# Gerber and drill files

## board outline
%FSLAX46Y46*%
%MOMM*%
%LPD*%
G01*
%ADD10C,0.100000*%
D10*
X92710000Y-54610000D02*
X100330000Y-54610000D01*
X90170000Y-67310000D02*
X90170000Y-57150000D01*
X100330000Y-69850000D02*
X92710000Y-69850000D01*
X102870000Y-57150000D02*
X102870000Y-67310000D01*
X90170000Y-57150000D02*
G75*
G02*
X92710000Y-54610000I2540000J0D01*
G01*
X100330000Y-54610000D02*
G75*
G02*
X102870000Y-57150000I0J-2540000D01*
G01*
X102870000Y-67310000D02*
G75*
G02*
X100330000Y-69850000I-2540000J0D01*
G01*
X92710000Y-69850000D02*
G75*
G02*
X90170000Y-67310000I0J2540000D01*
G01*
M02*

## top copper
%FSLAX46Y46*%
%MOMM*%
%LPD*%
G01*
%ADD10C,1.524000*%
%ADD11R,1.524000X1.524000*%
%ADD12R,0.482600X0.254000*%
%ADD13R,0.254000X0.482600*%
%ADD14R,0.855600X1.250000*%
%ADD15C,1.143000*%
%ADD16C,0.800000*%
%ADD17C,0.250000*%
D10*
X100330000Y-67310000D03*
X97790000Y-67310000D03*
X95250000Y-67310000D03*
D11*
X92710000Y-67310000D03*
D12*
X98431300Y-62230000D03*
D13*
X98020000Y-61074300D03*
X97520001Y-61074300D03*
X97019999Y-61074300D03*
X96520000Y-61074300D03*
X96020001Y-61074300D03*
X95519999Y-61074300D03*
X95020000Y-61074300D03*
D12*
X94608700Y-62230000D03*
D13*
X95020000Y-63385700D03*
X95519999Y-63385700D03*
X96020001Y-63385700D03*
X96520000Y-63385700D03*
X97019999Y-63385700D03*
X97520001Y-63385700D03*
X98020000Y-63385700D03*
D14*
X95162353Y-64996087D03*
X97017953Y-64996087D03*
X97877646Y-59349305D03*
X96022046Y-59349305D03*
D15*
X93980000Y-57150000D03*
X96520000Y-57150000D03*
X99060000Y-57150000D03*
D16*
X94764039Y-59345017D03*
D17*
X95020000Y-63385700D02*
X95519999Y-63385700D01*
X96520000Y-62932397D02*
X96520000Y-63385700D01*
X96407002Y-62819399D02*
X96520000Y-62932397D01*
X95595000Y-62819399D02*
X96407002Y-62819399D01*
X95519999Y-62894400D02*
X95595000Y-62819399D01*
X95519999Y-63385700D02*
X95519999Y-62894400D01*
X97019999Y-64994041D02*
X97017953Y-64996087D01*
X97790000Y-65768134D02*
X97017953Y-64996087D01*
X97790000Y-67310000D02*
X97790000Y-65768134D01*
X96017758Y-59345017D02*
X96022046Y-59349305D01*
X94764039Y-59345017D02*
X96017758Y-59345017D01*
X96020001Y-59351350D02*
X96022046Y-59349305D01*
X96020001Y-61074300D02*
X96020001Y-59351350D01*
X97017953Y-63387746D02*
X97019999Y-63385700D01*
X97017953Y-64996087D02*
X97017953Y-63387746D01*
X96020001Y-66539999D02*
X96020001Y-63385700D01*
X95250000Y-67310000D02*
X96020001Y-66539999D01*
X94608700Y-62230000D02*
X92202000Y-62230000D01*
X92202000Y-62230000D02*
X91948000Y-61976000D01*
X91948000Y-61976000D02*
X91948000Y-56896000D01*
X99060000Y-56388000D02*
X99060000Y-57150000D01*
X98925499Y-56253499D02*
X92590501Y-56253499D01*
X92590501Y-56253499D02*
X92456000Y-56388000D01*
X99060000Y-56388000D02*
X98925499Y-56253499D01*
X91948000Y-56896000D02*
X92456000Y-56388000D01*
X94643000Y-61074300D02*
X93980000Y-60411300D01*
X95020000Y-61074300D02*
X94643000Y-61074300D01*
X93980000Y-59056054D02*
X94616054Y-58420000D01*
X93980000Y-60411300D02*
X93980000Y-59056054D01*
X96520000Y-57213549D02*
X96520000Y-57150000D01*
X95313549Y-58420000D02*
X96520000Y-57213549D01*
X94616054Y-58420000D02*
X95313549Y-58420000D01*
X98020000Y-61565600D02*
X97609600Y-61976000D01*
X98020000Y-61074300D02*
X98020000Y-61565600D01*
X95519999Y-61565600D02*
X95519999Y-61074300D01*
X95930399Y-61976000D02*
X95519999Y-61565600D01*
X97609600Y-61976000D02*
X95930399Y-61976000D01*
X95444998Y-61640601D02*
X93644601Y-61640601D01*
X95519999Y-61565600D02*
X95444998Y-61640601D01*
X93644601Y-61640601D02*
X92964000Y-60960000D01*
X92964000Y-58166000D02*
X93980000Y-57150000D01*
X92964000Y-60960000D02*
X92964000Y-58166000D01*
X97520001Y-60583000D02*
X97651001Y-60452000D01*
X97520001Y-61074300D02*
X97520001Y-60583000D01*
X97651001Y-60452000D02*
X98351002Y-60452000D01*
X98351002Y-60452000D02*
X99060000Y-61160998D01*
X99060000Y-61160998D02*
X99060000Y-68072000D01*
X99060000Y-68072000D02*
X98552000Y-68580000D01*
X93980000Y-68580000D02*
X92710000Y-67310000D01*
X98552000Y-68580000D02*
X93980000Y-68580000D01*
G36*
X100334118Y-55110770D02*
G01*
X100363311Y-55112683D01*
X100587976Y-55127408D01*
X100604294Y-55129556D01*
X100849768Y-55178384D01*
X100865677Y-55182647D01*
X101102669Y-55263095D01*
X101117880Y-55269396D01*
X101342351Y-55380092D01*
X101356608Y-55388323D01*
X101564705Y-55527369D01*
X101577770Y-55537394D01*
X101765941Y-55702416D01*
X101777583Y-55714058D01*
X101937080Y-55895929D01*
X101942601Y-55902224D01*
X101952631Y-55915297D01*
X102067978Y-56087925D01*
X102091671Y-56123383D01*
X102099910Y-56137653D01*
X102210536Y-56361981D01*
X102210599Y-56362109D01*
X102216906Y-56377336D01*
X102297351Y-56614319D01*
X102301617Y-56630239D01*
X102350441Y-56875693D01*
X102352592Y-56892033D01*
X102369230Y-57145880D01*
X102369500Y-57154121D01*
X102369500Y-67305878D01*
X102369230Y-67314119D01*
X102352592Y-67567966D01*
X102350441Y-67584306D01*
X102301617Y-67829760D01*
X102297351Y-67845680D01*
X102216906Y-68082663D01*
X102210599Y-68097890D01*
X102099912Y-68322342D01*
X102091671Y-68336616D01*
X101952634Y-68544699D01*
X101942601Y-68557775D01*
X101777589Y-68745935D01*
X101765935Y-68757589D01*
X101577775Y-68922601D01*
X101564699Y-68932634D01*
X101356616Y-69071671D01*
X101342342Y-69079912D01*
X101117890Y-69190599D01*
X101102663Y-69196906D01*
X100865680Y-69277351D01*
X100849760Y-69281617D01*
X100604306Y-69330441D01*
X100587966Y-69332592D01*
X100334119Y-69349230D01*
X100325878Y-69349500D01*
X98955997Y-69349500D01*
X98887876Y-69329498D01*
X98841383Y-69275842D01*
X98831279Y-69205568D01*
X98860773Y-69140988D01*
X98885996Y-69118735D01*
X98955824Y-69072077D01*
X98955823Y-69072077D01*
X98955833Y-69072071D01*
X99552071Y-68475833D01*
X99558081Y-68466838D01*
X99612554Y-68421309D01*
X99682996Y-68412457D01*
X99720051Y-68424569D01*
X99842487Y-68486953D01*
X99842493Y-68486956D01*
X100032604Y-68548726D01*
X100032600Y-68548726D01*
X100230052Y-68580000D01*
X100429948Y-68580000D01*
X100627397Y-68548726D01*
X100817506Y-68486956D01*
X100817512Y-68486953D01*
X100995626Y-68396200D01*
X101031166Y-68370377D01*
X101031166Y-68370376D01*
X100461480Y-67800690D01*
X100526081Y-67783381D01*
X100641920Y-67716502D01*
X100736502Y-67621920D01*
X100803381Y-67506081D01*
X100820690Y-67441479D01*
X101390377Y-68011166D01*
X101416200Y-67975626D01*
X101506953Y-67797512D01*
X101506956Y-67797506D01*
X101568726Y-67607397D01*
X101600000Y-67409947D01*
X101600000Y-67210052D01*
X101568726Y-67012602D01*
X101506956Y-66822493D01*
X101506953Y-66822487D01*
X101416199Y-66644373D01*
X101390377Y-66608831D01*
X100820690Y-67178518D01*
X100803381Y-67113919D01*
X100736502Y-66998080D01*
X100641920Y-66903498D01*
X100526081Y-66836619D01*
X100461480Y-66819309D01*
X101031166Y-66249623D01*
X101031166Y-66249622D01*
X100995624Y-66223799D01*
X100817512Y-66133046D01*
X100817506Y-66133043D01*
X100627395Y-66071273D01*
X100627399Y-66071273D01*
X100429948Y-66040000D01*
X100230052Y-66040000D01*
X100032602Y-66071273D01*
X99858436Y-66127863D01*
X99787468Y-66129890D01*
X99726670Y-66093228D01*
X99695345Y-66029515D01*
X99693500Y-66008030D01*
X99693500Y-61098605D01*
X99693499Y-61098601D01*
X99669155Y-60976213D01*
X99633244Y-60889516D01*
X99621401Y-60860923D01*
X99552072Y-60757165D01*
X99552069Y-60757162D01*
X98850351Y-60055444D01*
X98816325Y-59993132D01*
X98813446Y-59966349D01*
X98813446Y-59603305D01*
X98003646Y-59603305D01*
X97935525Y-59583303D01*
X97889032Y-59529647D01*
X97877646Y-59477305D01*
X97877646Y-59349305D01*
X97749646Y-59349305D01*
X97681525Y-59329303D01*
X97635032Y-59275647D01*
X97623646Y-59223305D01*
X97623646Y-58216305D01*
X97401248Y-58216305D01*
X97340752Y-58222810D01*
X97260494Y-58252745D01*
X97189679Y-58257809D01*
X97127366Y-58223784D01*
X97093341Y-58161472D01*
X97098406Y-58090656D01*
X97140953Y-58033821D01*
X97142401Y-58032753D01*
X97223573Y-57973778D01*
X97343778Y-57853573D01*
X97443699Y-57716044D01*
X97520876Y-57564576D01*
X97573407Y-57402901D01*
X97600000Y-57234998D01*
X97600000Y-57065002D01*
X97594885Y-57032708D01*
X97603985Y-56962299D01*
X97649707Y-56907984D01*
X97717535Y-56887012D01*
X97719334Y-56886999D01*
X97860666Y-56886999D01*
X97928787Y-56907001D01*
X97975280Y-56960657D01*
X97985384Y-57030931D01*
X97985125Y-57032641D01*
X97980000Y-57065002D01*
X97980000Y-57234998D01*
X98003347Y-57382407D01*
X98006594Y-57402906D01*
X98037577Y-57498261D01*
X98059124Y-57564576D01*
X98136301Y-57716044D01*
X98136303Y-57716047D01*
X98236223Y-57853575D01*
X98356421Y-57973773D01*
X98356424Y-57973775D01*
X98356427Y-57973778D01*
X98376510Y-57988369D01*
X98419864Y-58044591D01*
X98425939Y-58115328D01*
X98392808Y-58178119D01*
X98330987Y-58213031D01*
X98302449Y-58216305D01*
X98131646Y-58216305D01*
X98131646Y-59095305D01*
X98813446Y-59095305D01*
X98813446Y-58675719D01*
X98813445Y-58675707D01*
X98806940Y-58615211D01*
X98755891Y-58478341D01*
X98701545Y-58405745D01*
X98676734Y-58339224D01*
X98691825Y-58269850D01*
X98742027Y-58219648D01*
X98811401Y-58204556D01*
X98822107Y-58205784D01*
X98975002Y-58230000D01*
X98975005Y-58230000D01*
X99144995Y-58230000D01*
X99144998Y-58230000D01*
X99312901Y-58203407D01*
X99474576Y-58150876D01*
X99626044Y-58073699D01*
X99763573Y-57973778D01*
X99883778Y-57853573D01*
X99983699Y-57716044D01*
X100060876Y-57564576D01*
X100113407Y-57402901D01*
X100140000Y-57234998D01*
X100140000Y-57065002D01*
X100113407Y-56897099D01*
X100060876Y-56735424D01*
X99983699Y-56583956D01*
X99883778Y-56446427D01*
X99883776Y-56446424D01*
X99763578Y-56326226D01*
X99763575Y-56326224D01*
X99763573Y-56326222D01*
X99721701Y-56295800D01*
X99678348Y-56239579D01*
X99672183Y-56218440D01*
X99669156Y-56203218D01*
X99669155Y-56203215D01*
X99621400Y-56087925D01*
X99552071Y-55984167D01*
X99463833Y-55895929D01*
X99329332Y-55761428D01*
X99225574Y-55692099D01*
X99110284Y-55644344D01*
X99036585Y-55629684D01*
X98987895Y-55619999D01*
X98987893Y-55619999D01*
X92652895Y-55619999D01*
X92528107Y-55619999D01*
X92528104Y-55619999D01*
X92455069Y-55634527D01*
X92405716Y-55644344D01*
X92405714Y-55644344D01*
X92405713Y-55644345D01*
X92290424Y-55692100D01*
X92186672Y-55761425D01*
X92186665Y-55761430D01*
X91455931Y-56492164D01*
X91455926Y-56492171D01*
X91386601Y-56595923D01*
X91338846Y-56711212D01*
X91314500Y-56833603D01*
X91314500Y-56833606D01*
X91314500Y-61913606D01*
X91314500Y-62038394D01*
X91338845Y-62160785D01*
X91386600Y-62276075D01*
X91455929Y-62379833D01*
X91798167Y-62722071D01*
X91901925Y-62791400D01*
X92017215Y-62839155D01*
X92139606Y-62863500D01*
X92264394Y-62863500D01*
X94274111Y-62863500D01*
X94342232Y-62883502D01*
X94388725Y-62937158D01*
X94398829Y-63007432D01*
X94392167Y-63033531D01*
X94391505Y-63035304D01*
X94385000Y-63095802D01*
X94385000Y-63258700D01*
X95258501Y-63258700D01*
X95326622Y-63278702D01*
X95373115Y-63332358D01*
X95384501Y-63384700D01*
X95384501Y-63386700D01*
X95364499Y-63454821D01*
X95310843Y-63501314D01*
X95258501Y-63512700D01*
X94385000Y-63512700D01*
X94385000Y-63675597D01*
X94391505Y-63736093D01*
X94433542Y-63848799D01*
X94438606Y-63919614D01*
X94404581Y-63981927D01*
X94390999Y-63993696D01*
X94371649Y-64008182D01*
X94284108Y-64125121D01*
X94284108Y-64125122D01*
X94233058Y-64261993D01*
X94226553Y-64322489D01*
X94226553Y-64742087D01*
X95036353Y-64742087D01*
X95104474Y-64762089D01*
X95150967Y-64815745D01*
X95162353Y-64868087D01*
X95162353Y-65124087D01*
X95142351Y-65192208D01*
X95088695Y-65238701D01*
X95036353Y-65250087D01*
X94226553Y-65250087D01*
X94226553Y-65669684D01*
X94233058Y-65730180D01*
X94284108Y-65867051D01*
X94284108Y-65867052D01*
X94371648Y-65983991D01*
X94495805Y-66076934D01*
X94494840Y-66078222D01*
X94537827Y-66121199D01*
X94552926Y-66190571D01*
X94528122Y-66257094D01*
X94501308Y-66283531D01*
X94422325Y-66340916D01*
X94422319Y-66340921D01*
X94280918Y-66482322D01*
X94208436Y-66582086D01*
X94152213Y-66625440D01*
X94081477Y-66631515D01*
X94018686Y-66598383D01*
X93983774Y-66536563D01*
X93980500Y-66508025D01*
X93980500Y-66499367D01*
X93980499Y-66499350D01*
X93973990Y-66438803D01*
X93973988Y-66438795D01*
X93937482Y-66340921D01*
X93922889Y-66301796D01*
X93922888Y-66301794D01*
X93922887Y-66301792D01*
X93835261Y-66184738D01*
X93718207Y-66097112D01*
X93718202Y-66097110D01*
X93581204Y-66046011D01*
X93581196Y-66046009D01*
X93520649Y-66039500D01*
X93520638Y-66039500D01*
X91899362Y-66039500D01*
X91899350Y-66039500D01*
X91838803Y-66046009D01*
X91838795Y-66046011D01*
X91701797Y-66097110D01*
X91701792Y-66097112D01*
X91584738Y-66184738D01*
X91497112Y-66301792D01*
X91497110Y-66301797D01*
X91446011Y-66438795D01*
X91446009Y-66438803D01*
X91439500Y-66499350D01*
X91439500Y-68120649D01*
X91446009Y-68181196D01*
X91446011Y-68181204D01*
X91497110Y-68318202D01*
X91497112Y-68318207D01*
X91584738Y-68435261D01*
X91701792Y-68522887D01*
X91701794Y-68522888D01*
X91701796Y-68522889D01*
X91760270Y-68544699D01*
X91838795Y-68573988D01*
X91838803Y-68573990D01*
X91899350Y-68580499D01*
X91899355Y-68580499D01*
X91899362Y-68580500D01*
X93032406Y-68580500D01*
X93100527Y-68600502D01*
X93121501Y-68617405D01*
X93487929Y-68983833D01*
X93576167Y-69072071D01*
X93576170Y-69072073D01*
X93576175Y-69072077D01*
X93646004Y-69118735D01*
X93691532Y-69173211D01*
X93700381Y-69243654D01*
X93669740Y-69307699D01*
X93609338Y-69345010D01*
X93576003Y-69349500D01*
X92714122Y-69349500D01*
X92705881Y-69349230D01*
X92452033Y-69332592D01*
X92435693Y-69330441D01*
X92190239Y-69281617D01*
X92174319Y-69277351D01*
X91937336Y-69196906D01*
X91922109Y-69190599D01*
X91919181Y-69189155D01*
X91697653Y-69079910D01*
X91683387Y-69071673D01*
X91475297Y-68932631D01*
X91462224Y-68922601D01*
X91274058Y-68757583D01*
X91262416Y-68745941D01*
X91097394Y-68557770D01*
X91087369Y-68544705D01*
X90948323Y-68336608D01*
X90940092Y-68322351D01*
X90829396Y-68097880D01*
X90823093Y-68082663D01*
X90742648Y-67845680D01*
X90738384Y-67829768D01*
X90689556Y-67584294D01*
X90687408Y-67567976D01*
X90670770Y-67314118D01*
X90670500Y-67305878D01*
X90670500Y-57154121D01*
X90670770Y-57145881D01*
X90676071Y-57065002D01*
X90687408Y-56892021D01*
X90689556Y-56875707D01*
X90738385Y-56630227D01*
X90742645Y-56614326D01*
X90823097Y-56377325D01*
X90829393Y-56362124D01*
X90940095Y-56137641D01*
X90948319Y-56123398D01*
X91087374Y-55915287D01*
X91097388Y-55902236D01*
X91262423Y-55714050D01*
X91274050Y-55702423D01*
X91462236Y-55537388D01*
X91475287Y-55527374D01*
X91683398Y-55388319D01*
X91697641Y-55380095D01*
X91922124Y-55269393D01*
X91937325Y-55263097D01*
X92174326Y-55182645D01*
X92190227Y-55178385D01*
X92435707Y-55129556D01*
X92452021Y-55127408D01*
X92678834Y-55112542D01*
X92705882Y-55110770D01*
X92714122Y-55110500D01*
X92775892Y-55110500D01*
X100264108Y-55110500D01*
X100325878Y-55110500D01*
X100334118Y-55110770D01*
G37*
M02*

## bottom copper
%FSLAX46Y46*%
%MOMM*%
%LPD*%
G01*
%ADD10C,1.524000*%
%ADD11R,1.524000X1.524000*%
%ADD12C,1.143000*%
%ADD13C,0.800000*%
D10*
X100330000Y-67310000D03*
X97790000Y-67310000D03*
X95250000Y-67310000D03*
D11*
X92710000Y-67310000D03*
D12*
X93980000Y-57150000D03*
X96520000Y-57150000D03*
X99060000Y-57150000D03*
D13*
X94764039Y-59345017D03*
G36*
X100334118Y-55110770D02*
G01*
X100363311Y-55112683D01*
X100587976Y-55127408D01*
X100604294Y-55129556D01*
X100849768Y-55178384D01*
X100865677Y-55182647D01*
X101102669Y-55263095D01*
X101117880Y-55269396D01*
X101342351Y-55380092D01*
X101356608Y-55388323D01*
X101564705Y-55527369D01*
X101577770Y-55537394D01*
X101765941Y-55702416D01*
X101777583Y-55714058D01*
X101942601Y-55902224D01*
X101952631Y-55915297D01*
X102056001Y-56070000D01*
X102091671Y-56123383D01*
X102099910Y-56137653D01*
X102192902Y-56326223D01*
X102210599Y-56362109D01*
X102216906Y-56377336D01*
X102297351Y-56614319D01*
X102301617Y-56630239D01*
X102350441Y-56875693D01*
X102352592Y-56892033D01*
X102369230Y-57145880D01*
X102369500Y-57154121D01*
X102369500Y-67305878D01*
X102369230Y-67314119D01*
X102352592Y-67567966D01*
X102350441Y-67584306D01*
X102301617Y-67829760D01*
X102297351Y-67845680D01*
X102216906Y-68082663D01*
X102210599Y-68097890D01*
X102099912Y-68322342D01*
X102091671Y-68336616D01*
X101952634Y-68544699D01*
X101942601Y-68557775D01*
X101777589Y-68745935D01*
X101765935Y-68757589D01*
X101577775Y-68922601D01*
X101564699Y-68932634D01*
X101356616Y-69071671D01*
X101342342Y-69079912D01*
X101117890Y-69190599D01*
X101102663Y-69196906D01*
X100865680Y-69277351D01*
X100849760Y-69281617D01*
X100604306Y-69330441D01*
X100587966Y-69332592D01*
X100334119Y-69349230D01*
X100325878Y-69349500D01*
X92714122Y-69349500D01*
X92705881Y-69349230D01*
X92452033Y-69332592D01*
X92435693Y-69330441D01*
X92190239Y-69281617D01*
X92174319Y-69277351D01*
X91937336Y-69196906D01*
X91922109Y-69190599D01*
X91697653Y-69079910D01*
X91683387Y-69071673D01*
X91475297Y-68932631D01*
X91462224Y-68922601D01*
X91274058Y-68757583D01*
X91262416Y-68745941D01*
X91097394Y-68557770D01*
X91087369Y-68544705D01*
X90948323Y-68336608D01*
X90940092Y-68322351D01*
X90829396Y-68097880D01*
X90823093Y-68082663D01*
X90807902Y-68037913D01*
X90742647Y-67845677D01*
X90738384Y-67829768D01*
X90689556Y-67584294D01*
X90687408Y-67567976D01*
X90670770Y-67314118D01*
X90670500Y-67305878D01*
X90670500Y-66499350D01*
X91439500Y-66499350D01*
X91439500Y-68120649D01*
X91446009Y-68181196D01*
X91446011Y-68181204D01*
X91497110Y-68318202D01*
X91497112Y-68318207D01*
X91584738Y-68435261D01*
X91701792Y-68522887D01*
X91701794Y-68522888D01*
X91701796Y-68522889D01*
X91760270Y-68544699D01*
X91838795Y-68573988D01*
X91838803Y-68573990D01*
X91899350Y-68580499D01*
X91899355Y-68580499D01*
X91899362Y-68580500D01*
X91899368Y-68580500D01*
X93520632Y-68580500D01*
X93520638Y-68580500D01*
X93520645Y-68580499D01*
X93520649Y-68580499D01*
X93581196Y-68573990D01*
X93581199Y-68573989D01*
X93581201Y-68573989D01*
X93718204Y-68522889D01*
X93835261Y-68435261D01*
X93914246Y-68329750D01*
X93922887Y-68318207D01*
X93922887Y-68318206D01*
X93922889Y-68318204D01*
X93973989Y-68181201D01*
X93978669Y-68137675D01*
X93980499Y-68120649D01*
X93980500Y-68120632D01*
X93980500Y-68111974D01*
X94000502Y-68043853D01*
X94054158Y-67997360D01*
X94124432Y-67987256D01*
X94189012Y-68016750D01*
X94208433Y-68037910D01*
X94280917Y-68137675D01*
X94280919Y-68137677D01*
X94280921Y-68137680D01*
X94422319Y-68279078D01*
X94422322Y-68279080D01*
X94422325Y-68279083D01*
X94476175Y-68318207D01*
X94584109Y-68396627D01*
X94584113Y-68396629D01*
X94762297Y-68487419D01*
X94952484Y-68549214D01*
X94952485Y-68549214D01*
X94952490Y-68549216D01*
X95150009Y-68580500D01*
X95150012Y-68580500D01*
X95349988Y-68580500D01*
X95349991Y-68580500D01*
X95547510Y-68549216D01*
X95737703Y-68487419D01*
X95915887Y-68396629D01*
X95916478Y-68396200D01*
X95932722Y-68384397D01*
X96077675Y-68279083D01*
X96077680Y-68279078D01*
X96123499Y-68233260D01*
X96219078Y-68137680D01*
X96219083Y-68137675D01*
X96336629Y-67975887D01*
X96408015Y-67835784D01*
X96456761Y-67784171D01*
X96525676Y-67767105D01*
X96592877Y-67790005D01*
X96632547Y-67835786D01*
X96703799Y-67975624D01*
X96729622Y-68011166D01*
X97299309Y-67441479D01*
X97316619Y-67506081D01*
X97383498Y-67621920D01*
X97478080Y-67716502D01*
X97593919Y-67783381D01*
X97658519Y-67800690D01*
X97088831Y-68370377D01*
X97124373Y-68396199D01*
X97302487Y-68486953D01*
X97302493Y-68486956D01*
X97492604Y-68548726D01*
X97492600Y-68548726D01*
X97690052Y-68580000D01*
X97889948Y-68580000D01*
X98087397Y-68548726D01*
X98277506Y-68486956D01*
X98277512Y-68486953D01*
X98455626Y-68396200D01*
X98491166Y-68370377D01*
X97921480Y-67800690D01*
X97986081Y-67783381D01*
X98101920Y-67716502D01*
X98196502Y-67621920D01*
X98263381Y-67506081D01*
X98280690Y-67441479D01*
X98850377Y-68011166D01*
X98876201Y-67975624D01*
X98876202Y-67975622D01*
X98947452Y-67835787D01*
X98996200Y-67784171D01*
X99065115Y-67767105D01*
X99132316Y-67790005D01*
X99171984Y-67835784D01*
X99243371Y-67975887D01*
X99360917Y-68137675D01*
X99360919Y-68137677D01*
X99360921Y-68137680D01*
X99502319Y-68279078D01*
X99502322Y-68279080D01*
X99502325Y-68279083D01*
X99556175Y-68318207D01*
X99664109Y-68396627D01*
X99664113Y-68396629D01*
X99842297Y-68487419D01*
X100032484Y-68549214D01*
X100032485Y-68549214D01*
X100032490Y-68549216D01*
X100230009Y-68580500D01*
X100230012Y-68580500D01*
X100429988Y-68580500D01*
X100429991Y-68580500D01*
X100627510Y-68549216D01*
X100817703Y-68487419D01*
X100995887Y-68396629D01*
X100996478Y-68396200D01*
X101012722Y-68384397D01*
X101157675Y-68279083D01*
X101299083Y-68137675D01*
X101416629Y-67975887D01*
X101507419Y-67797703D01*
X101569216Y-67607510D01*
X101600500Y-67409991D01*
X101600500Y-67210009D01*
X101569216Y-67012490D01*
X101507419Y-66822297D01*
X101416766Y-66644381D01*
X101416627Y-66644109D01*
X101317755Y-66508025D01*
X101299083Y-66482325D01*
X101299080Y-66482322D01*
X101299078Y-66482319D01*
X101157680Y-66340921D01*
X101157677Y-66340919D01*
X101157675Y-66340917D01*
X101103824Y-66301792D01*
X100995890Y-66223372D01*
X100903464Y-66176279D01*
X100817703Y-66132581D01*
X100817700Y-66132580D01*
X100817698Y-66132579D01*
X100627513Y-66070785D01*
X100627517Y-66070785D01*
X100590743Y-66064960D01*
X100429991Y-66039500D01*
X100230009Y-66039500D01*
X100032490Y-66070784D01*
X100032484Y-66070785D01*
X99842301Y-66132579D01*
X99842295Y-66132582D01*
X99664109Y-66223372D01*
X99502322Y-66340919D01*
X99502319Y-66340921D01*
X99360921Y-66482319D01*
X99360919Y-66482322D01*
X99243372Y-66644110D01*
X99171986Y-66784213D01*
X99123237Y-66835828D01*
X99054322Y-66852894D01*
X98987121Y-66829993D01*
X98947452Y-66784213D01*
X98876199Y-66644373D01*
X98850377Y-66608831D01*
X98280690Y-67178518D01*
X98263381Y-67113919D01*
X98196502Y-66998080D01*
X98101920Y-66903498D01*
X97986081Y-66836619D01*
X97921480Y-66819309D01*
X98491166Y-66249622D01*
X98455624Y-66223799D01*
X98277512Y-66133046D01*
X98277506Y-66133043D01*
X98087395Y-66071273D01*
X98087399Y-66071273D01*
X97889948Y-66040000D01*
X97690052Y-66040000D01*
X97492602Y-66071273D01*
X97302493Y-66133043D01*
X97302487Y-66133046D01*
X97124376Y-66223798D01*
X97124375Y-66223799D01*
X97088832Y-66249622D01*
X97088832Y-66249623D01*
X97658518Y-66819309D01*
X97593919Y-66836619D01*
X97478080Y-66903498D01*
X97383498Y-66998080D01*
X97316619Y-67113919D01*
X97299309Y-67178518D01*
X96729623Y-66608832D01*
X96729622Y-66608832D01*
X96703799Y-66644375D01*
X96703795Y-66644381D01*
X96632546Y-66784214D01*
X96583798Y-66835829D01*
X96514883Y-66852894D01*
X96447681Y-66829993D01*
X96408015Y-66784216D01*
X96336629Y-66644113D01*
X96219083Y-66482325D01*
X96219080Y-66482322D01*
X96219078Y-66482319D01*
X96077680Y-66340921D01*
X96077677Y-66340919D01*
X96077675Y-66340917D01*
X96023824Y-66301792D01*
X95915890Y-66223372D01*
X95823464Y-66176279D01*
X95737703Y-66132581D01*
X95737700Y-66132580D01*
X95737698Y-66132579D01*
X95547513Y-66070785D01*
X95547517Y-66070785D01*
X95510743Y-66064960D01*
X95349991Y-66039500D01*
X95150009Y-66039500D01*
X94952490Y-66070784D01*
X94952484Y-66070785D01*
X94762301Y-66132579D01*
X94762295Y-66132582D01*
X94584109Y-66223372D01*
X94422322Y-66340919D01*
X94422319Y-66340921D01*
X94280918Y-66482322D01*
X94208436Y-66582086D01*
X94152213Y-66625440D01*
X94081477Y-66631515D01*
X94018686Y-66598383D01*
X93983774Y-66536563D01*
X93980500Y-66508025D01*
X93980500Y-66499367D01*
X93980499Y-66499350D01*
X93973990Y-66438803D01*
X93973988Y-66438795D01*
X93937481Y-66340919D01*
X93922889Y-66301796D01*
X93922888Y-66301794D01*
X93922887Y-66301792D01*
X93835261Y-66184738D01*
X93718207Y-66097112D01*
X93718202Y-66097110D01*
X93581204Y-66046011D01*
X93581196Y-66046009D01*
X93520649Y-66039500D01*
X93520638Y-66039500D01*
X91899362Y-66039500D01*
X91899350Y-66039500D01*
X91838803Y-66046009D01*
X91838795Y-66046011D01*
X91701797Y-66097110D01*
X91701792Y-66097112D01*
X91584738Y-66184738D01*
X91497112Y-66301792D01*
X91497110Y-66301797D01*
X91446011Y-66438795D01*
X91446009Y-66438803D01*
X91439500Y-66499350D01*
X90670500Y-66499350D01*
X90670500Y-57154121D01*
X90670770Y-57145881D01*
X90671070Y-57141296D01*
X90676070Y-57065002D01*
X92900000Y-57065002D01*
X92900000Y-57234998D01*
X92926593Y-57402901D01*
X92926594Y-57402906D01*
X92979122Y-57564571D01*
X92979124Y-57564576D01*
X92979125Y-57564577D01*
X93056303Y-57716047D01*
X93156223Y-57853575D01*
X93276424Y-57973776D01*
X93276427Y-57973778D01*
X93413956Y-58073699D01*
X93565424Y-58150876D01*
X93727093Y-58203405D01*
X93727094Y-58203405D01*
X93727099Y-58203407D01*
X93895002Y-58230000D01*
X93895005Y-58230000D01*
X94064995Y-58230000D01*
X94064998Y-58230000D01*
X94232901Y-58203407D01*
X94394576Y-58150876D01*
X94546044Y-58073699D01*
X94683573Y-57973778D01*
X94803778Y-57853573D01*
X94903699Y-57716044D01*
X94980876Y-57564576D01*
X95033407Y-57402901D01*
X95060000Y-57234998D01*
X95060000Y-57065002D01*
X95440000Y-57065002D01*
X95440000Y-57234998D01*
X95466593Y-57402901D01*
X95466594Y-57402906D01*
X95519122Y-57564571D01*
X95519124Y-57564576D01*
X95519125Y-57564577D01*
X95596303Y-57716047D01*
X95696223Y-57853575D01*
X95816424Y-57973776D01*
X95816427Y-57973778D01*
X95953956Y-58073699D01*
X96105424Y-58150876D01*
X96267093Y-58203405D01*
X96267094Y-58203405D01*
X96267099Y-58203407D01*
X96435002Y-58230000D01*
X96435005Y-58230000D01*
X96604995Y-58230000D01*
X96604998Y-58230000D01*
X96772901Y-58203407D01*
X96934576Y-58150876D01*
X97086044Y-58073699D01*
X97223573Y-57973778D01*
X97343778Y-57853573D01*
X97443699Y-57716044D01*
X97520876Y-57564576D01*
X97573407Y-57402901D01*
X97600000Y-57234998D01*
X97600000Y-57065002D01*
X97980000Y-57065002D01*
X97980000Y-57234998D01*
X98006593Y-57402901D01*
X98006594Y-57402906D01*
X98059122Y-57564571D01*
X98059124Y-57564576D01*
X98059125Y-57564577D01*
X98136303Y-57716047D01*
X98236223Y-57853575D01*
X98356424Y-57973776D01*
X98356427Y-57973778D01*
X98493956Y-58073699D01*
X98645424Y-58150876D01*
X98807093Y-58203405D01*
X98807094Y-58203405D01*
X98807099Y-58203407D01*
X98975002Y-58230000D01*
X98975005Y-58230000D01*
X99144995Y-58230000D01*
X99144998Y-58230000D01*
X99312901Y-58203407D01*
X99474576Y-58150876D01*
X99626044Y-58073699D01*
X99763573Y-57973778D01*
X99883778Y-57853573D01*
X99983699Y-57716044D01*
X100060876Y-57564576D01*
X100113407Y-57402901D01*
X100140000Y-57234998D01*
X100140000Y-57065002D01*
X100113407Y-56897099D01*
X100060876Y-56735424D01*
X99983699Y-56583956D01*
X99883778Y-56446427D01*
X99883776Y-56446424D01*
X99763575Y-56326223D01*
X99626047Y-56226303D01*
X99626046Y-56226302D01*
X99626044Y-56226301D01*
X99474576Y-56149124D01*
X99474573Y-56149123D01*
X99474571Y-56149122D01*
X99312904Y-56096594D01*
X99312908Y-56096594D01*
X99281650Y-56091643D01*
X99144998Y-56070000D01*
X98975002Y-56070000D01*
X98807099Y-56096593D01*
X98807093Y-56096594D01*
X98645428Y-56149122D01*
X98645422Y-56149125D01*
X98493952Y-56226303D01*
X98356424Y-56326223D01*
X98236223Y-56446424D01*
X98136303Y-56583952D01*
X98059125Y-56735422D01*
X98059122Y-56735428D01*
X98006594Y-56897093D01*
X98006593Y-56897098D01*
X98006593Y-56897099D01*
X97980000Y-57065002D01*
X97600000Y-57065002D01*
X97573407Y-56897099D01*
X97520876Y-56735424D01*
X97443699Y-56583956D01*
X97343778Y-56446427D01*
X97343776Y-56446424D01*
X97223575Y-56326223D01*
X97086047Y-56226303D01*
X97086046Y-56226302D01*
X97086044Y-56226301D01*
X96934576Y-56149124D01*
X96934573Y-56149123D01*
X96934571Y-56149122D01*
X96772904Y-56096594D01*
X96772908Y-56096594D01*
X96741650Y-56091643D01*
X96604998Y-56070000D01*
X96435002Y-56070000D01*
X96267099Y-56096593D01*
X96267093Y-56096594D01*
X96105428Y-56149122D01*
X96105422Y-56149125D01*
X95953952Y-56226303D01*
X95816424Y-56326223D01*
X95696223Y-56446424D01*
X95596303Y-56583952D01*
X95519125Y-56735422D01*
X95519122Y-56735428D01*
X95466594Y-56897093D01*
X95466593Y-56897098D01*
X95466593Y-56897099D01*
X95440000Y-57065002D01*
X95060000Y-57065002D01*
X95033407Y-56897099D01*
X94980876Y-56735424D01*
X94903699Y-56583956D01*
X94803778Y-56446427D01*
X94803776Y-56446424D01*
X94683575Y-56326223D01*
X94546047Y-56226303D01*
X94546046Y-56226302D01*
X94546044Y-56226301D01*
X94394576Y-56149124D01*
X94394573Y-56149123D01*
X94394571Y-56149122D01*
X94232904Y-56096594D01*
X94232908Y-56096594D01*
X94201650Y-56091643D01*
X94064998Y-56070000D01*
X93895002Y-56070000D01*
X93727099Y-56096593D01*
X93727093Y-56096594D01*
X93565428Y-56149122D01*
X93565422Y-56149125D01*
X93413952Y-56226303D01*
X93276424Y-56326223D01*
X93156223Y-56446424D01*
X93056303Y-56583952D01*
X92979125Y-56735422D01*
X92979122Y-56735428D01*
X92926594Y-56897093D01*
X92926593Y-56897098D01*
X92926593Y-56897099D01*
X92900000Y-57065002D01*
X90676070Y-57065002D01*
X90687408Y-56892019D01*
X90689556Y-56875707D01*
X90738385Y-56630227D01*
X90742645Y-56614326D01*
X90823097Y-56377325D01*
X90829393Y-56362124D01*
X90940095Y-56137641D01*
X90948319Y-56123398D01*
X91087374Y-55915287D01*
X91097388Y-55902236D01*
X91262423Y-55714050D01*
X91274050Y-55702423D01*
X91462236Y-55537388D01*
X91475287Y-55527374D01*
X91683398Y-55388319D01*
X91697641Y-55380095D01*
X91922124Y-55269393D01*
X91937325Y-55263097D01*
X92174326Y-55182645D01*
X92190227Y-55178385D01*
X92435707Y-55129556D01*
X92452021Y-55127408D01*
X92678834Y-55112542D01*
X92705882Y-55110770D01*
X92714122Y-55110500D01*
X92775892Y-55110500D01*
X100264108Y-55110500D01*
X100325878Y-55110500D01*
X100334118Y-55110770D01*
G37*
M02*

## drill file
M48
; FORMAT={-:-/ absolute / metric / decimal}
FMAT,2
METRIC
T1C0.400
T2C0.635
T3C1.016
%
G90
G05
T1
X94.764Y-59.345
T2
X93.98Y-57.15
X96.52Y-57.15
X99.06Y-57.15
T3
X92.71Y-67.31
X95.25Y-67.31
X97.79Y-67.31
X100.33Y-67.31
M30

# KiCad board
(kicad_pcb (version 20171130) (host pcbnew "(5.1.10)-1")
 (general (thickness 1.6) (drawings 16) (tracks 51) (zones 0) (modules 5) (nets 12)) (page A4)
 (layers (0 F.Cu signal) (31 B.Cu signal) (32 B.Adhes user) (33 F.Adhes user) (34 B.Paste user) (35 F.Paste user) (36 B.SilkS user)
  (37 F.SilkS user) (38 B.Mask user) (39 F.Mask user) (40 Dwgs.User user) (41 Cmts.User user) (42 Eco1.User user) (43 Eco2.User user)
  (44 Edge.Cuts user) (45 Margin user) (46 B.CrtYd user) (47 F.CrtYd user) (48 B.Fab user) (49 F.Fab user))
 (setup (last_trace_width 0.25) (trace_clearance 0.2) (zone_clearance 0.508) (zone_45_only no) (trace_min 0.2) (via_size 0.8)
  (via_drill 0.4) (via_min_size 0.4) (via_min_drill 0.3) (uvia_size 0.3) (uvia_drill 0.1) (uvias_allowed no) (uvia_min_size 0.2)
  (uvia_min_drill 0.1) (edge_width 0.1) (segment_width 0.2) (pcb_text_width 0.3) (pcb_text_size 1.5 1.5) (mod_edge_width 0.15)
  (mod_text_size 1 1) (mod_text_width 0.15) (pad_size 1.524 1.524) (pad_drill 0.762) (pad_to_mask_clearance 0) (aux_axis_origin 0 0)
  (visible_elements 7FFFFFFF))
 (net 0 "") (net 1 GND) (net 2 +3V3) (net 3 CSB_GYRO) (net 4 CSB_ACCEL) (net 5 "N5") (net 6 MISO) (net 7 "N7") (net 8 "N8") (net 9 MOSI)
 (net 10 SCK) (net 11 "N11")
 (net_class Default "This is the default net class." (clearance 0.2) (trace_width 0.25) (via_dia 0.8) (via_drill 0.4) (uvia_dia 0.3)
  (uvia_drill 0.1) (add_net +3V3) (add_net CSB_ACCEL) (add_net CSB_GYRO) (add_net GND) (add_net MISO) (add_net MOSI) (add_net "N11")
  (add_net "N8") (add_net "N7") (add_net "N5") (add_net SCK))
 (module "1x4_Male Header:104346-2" (layer F.Cu) (at 92.71 67.31 180)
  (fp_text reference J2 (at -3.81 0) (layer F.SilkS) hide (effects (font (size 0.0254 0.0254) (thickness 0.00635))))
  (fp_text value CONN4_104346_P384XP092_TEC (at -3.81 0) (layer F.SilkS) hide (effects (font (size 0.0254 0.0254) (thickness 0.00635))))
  (pad 4 thru_hole circle (at -7.62 0 180) (size 1.524 1.524) (drill 1.016) (layers *.Cu *.Mask) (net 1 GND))
  (pad 3 thru_hole circle (at -5.08 0 180) (size 1.524 1.524) (drill 1.016) (layers *.Cu *.Mask) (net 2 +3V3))
  (pad 2 thru_hole circle (at -2.54 0 180) (size 1.524 1.524) (drill 1.016) (layers *.Cu *.Mask) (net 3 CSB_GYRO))
  (pad 1 thru_hole rect (at 0 0 180) (size 1.524 1.524) (drill 1.016) (layers *.Cu *.Mask) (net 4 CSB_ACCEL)))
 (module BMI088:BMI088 (layer F.Cu) (at 96.52 62.23 180)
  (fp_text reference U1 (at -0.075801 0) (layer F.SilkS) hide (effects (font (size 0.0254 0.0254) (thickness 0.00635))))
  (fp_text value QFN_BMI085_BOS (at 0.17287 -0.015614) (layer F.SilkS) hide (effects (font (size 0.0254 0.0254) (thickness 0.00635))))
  (pad 16 smd rect (at -1.9113 0 270) (size 0.254 0.4826) (layers F.Cu F.Paste F.Mask) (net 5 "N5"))
  (pad 15 smd rect (at -1.5 1.1557 180) (size 0.254 0.4826) (layers F.Cu F.Paste F.Mask) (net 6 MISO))
  (pad 14 smd rect (at -1.000001 1.1557 180) (size 0.254 0.4826) (layers F.Cu F.Paste F.Mask) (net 4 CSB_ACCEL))
  (pad 13 smd rect (at -0.499999 1.1557 180) (size 0.254 0.4826) (layers F.Cu F.Paste F.Mask) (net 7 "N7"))
  (pad 12 smd rect (at 0 1.1557 180) (size 0.254 0.4826) (layers F.Cu F.Paste F.Mask) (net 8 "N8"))
  (pad 11 smd rect (at 0.499999 1.1557 180) (size 0.254 0.4826) (layers F.Cu F.Paste F.Mask) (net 2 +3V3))
  (pad 10 smd rect (at 1.000001 1.1557 180) (size 0.254 0.4826) (layers F.Cu F.Paste F.Mask) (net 6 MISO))
  (pad 9 smd rect (at 1.5 1.1557 180) (size 0.254 0.4826) (layers F.Cu F.Paste F.Mask) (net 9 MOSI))
  (pad 8 smd rect (at 1.9113 0 270) (size 0.254 0.4826) (layers F.Cu F.Paste F.Mask) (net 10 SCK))
  (pad 7 smd rect (at 1.5 -1.1557 180) (size 0.254 0.4826) (layers F.Cu F.Paste F.Mask) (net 1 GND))
  (pad 6 smd rect (at 1.000001 -1.1557 180) (size 0.254 0.4826) (layers F.Cu F.Paste F.Mask) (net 1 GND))
  (pad 5 smd rect (at 0.499999 -1.1557 180) (size 0.254 0.4826) (layers F.Cu F.Paste F.Mask) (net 3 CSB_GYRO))
  (pad 4 smd rect (at 0 -1.1557 180) (size 0.254 0.4826) (layers F.Cu F.Paste F.Mask) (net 1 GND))
  (pad 3 smd rect (at -0.499999 -1.1557 180) (size 0.254 0.4826) (layers F.Cu F.Paste F.Mask) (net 2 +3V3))
  (pad 2 smd rect (at -1.000001 -1.1557 180) (size 0.254 0.4826) (layers F.Cu F.Paste F.Mask))
  (pad 1 smd rect (at -1.5 -1.1557 180) (size 0.254 0.4826) (layers F.Cu F.Paste F.Mask) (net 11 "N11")))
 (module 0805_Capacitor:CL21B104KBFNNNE (layer F.Cu) (at 96.090153 64.996087 180)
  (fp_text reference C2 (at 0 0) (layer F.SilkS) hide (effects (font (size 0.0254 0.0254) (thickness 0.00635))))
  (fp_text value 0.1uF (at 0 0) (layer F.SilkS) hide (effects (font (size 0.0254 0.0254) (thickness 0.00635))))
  (pad 2 smd rect (at 0.9278 0 180) (size 0.8556 1.25) (layers F.Cu F.Paste F.Mask) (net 1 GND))
  (pad 1 smd rect (at -0.9278 0 180) (size 0.8556 1.25) (layers F.Cu F.Paste F.Mask) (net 2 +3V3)))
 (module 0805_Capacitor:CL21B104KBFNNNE (layer F.Cu) (at 96.949846 59.349305)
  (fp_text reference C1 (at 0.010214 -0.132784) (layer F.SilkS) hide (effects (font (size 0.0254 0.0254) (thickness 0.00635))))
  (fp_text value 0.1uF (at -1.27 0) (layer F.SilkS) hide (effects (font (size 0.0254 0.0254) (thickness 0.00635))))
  (pad 2 smd rect (at 0.9278 0) (size 0.8556 1.25) (layers F.Cu F.Paste F.Mask) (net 1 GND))
  (pad 1 smd rect (at -0.9278 0) (size 0.8556 1.25) (layers F.Cu F.Paste F.Mask) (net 2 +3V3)))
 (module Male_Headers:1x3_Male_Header (layer F.Cu) (at 99.06 57.15 180)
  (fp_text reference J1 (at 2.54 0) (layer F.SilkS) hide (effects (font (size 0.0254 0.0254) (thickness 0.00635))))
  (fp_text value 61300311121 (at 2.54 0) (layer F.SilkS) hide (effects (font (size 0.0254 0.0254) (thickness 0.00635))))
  (pad 3 thru_hole circle (at 5.08 0 180) (size 1.143 1.143) (drill 0.635) (layers *.Cu *.Mask) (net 6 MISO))
  (pad 2 thru_hole circle (at 2.54 0 180) (size 1.143 1.143) (drill 0.635) (layers *.Cu *.Mask) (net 9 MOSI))
  (pad 1 thru_hole circle (at 0 0 180) (size 1.143 1.143) (drill 0.635) (layers *.Cu *.Mask) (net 10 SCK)))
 (gr_line (start 92.71 54.61) (end 100.33 54.61) (layer Edge.Cuts) (width 0.1))
 (gr_line (start 90.17 67.31) (end 90.17 57.15) (layer Edge.Cuts) (width 0.1))
 (gr_line (start 100.33 69.85) (end 92.71 69.85) (layer Edge.Cuts) (width 0.1))
 (gr_line (start 102.87 57.15) (end 102.87 67.31) (layer Edge.Cuts) (width 0.1))
 (gr_arc (start 92.71 57.15) (end 92.71 54.61) (angle -90) (layer Edge.Cuts) (width 0.1))
 (gr_arc (start 100.33 57.15) (end 102.87 57.15) (angle -90) (layer Edge.Cuts) (width 0.1))
 (gr_arc (start 100.33 67.31) (end 100.33 69.85) (angle -90) (layer Edge.Cuts) (width 0.1))
 (gr_arc (start 92.71 67.31) (end 90.17 67.31) (angle -90) (layer Edge.Cuts) (width 0.1))
 (segment (start 95.02 63.3857) (end 95.519999 63.3857) (width 0.25) (layer F.Cu) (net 1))
 (segment (start 96.52 62.932397) (end 96.52 63.3857) (width 0.25) (layer F.Cu) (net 1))
 (segment (start 96.407002 62.819399) (end 96.52 62.932397) (width 0.25) (layer F.Cu) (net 1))
 (segment (start 95.595 62.819399) (end 96.407002 62.819399) (width 0.25) (layer F.Cu) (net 1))
 (segment (start 95.519999 62.8944) (end 95.595 62.819399) (width 0.25) (layer F.Cu) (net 1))
 (segment (start 95.519999 63.3857) (end 95.519999 62.8944) (width 0.25) (layer F.Cu) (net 1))
 (segment (start 97.019999 64.994041) (end 97.017953 64.996087) (width 0.25) (layer F.Cu) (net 2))
 (segment (start 97.79 65.768134) (end 97.017953 64.996087) (width 0.25) (layer F.Cu) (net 2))
 (segment (start 97.79 67.31) (end 97.79 65.768134) (width 0.25) (layer F.Cu) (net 2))
 (via (at 94.764039 59.345017) (size 0.8) (drill 0.4) (layers F.Cu B.Cu) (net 2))
 (segment (start 96.017758 59.345017) (end 96.022046 59.349305) (width 0.25) (layer F.Cu) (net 2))
 (segment (start 94.764039 59.345017) (end 96.017758 59.345017) (width 0.25) (layer F.Cu) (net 2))
 (segment (start 96.020001 59.35135) (end 96.022046 59.349305) (width 0.25) (layer F.Cu) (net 2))
 (segment (start 96.020001 61.0743) (end 96.020001 59.35135) (width 0.25) (layer F.Cu) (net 2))
 (segment (start 97.017953 63.387746) (end 97.019999 63.3857) (width 0.25) (layer F.Cu) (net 2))
 (segment (start 97.017953 64.996087) (end 97.017953 63.387746) (width 0.25) (layer F.Cu) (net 2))
 (segment (start 96.020001 66.539999) (end 96.020001 63.3857) (width 0.25) (layer F.Cu) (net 3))
 (segment (start 95.25 67.31) (end 96.020001 66.539999) (width 0.25) (layer F.Cu) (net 3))
 (segment (start 94.6087 62.23) (end 92.202 62.23) (width 0.25) (layer F.Cu) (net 10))
 (segment (start 92.202 62.23) (end 91.948 61.976) (width 0.25) (layer F.Cu) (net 10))
 (segment (start 91.948 61.976) (end 91.948 56.896) (width 0.25) (layer F.Cu) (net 10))
 (segment (start 99.06 56.388) (end 99.06 57.15) (width 0.25) (layer F.Cu) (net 10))
 (segment (start 98.925499 56.253499) (end 92.590501 56.253499) (width 0.25) (layer F.Cu) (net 10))
 (segment (start 92.590501 56.253499) (end 92.456 56.388) (width 0.25) (layer F.Cu) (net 10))
 (segment (start 99.06 56.388) (end 98.925499 56.253499) (width 0.25) (layer F.Cu) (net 10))
 (segment (start 91.948 56.896) (end 92.456 56.388) (width 0.25) (layer F.Cu) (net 10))
 (segment (start 94.643 61.0743) (end 93.98 60.4113) (width 0.25) (layer F.Cu) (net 9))
 (segment (start 95.02 61.0743) (end 94.643 61.0743) (width 0.25) (layer F.Cu) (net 9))
 (segment (start 93.98 59.056054) (end 94.616054 58.42) (width 0.25) (layer F.Cu) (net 9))
 (segment (start 93.98 60.4113) (end 93.98 59.056054) (width 0.25) (layer F.Cu) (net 9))
 (segment (start 96.52 57.213549) (end 96.52 57.15) (width 0.25) (layer F.Cu) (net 9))
 (segment (start 95.313549 58.42) (end 96.52 57.213549) (width 0.25) (layer F.Cu) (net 9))
 (segment (start 94.616054 58.42) (end 95.313549 58.42) (width 0.25) (layer F.Cu) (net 9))
 (segment (start 98.02 61.5656) (end 97.6096 61.976) (width 0.25) (layer F.Cu) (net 6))
 (segment (start 98.02 61.0743) (end 98.02 61.5656) (width 0.25) (layer F.Cu) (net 6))
 (segment (start 95.519999 61.5656) (end 95.519999 61.0743) (width 0.25) (layer F.Cu) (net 6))
 (segment (start 95.930399 61.976) (end 95.519999 61.5656) (width 0.25) (layer F.Cu) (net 6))
 (segment (start 97.6096 61.976) (end 95.930399 61.976) (width 0.25) (layer F.Cu) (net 6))
 (segment (start 95.444998 61.640601) (end 93.644601 61.640601) (width 0.25) (layer F.Cu) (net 6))
 (segment (start 95.519999 61.5656) (end 95.444998 61.640601) (width 0.25) (layer F.Cu) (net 6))
 (segment (start 93.644601 61.640601) (end 92.964 60.96) (width 0.25) (layer F.Cu) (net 6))
 (segment (start 92.964 58.166) (end 93.98 57.15) (width 0.25) (layer F.Cu) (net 6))
 (segment (start 92.964 60.96) (end 92.964 58.166) (width 0.25) (layer F.Cu) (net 6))
 (segment (start 97.520001 60.583) (end 97.651001 60.452) (width 0.25) (layer F.Cu) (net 4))
 (segment (start 97.520001 61.0743) (end 97.520001 60.583) (width 0.25) (layer F.Cu) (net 4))
 (segment (start 97.651001 60.452) (end 98.351002 60.452) (width 0.25) (layer F.Cu) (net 4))
 (segment (start 98.351002 60.452) (end 99.06 61.160998) (width 0.25) (layer F.Cu) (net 4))
 (segment (start 99.06 61.160998) (end 99.06 68.072) (width 0.25) (layer F.Cu) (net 4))
 (segment (start 99.06 68.072) (end 98.552 68.58) (width 0.25) (layer F.Cu) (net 4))
 (segment (start 93.98 68.58) (end 92.71 67.31) (width 0.25) (layer F.Cu) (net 4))
 (segment (start 98.552 68.58) (end 93.98 68.58) (width 0.25) (layer F.Cu) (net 4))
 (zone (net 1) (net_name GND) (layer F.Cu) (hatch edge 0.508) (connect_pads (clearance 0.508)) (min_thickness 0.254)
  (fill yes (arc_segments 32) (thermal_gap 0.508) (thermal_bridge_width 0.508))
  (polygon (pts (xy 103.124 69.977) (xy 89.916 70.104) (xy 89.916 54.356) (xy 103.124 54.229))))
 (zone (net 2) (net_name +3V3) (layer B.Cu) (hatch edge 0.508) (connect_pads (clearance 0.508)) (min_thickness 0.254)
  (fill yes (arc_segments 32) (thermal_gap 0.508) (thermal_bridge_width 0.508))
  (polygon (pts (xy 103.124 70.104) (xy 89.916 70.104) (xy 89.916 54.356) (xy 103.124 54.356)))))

